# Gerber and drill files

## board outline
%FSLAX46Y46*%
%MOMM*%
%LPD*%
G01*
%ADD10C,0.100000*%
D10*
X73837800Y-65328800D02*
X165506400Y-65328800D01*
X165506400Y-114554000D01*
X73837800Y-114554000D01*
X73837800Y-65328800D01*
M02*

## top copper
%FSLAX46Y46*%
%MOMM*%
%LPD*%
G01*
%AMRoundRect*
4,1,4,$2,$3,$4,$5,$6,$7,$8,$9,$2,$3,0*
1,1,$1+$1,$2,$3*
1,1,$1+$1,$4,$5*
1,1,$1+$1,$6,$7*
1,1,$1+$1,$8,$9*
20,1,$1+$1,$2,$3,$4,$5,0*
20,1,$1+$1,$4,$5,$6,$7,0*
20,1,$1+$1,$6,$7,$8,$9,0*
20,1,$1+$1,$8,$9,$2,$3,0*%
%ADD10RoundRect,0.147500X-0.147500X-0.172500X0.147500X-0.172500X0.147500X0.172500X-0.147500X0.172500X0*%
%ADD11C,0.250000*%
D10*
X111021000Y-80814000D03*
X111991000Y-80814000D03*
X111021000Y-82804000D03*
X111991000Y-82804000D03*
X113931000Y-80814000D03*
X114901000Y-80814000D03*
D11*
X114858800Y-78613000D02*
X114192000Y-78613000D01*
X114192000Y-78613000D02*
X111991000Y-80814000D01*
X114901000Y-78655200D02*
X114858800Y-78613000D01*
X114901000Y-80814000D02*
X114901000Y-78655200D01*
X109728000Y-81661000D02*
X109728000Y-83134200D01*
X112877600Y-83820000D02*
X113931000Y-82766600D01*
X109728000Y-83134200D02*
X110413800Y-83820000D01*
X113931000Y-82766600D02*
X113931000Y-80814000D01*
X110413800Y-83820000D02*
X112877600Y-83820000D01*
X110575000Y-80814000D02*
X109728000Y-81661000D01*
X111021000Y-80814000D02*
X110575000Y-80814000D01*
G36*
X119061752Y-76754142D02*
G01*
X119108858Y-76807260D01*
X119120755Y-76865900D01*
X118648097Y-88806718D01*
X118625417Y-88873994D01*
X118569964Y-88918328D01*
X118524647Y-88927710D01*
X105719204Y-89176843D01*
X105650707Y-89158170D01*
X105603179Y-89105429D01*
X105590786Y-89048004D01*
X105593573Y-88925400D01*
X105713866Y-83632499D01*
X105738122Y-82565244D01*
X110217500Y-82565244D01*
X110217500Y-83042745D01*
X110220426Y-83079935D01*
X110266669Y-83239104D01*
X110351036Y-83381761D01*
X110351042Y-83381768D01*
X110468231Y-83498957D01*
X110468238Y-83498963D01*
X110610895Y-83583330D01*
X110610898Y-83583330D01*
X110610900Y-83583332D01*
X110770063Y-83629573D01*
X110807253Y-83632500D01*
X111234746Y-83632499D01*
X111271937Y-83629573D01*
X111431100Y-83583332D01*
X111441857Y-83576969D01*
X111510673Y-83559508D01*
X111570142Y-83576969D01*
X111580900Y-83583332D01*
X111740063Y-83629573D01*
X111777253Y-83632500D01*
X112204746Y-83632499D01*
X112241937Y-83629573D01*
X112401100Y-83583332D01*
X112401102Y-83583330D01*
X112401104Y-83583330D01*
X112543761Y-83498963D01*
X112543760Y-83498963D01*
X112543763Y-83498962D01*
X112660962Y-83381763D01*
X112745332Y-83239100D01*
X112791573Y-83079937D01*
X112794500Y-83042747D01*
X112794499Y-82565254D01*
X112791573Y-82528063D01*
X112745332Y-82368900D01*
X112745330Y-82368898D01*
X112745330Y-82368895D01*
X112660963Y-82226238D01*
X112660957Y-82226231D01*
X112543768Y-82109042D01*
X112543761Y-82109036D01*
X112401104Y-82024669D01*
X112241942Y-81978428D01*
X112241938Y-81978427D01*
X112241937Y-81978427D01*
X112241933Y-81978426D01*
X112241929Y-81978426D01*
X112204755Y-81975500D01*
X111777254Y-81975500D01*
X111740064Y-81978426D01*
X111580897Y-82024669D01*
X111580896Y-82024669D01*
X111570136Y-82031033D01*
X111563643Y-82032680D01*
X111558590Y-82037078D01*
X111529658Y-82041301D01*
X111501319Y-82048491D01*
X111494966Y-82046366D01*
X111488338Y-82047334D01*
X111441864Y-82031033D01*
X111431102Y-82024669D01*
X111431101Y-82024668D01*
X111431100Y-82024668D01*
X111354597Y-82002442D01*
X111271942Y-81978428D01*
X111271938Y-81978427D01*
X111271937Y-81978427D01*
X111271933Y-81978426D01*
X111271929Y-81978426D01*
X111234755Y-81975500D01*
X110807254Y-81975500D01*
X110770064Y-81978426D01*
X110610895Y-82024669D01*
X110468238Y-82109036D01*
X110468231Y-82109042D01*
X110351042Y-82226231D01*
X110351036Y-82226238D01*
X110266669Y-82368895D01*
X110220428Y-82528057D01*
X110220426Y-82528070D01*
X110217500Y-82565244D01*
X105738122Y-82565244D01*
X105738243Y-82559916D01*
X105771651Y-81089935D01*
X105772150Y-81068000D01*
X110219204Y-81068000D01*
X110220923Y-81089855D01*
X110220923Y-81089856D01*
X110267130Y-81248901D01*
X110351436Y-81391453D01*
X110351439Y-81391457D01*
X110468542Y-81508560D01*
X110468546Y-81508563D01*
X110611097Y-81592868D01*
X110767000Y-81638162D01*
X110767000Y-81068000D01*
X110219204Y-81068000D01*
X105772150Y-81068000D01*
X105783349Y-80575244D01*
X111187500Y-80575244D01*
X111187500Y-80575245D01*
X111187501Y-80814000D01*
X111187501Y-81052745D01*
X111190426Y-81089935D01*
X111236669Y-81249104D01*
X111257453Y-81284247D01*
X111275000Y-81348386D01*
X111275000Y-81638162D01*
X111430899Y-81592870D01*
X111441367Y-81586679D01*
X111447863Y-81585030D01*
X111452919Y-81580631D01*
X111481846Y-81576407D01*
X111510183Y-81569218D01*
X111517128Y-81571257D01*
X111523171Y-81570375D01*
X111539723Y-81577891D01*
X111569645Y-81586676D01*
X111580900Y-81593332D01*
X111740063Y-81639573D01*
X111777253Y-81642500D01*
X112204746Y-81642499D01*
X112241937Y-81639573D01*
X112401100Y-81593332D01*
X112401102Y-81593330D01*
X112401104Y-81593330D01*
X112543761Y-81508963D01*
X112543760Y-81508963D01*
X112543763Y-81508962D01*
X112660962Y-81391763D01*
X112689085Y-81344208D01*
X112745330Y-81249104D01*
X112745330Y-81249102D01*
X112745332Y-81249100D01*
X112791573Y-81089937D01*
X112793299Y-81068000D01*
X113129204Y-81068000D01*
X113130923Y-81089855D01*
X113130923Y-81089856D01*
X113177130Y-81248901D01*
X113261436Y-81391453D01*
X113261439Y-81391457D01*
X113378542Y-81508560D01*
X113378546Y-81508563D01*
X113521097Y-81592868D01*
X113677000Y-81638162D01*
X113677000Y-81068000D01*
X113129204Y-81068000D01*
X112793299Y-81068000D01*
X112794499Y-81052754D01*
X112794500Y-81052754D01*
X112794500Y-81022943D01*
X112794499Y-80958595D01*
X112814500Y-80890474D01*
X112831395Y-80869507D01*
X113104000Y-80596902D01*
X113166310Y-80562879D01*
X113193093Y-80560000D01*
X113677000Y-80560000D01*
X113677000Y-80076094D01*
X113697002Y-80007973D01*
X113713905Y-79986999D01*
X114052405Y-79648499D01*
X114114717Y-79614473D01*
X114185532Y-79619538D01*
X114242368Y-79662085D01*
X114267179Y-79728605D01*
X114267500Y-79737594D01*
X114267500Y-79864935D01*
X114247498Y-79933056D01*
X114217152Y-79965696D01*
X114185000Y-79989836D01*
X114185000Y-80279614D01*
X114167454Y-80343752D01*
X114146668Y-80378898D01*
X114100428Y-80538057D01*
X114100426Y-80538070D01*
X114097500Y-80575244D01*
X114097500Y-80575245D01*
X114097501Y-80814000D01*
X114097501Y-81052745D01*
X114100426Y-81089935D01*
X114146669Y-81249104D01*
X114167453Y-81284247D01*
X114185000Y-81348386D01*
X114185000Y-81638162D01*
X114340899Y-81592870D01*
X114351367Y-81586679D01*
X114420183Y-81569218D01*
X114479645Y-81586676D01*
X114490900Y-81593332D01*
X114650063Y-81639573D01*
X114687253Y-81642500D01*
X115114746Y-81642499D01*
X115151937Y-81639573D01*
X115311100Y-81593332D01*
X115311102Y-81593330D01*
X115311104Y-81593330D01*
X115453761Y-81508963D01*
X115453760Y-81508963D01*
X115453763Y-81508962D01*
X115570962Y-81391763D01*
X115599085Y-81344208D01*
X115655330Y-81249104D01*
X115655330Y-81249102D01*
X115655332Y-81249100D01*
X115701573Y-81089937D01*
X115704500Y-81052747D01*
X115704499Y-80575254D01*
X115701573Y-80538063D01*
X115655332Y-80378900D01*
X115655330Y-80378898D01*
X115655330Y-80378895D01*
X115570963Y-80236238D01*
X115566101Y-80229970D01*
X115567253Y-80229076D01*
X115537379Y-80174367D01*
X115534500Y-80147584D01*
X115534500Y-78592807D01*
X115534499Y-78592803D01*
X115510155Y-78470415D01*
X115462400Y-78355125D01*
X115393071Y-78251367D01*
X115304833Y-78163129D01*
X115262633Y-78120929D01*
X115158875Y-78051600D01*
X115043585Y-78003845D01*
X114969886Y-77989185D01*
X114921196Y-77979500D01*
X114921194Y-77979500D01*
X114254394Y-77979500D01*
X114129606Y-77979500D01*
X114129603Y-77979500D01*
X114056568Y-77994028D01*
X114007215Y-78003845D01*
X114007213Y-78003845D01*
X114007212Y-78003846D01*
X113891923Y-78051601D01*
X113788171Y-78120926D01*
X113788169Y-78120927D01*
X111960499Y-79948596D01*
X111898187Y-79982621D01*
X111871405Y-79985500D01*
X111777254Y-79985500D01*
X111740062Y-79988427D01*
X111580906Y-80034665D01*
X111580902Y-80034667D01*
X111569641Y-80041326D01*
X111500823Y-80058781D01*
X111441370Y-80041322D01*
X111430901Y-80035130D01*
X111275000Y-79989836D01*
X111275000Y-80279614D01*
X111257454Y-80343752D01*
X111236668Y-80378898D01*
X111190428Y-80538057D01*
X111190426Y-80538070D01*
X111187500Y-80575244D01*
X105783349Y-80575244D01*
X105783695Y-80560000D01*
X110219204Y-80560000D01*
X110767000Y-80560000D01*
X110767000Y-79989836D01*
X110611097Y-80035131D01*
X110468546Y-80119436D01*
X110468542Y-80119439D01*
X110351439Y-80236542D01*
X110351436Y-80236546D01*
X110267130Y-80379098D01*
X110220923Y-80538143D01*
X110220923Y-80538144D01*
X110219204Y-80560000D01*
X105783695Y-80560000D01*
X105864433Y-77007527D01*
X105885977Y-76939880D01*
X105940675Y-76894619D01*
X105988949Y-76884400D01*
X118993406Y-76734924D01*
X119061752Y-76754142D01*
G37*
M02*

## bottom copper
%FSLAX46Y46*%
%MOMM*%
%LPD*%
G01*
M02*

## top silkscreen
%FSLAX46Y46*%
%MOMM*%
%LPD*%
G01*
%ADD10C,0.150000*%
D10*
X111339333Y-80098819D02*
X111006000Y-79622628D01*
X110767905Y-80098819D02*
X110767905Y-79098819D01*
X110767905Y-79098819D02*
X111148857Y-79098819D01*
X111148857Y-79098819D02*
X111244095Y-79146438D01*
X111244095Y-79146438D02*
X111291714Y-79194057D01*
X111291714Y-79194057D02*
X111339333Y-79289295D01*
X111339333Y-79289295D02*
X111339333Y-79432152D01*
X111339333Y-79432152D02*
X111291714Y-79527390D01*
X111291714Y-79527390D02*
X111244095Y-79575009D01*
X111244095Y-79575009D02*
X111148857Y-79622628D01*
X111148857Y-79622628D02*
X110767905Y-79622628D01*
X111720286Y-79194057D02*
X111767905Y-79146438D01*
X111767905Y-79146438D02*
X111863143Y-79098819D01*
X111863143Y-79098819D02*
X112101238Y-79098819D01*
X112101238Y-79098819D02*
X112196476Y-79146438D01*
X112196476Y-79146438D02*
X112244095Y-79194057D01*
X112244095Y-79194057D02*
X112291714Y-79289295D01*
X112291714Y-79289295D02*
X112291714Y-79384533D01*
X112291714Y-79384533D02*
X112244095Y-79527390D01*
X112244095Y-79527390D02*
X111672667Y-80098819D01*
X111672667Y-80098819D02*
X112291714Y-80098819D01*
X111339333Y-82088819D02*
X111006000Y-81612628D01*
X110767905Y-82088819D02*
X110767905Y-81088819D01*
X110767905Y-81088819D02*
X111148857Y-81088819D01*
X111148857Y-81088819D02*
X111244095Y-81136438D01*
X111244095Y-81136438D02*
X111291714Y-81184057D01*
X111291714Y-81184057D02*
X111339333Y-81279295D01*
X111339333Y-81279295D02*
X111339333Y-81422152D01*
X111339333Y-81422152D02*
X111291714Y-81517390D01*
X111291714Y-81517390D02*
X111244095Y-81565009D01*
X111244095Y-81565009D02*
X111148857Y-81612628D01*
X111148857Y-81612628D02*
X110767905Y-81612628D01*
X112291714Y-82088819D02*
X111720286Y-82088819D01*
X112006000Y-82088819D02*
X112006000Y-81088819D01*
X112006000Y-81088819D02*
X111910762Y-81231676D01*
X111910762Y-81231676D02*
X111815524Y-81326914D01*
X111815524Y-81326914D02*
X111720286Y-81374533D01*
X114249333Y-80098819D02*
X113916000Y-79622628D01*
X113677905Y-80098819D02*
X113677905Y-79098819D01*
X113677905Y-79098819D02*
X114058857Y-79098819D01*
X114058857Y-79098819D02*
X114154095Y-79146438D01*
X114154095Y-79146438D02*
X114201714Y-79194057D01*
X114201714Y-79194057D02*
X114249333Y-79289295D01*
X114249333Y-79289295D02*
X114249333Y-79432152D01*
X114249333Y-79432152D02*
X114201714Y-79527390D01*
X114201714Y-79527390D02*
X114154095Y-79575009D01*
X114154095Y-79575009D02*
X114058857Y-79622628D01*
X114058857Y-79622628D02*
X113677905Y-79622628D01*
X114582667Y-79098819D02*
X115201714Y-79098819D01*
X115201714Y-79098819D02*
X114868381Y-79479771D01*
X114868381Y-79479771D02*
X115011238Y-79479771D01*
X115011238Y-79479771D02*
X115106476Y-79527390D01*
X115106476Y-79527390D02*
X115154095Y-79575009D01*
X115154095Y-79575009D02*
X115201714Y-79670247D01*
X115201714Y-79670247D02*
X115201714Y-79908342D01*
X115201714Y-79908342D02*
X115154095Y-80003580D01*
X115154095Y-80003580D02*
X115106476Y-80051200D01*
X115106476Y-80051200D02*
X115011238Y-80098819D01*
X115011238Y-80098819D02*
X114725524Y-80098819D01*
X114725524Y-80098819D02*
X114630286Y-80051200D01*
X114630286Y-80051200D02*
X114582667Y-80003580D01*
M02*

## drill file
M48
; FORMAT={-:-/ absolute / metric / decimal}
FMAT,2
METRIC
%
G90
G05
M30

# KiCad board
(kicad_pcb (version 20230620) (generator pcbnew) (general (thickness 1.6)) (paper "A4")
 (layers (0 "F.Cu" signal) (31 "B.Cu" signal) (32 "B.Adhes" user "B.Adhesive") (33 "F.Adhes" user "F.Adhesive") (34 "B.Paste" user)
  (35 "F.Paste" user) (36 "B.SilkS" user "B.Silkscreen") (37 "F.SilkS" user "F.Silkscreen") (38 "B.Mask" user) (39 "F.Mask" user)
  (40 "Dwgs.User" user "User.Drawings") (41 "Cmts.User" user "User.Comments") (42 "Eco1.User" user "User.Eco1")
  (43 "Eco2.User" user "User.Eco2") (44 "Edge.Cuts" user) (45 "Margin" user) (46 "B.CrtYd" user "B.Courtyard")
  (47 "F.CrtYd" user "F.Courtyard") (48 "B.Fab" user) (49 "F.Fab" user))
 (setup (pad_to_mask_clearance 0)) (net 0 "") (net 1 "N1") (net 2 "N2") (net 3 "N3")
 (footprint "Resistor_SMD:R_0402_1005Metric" (layer "F.Cu") (at 111.506 80.814)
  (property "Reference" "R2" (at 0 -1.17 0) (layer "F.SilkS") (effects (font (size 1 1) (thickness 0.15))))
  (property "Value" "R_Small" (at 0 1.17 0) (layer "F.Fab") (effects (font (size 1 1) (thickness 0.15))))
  (pad "1" smd roundrect (at -0.485 0) (size 0.59 0.64) (layers "F.Cu" "F.Paste" "F.Mask") (roundrect_rratio 0.25) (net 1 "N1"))
  (pad "2" smd roundrect (at 0.485 0) (size 0.59 0.64) (layers "F.Cu" "F.Paste" "F.Mask") (roundrect_rratio 0.25) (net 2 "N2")))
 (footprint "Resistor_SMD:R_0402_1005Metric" (layer "F.Cu") (at 111.506 82.804)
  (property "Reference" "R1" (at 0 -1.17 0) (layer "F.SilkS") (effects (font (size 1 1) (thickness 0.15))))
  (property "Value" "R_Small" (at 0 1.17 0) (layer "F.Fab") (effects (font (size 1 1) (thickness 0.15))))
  (pad "1" smd roundrect (at -0.485 0) (size 0.59 0.64) (layers "F.Cu" "F.Paste" "F.Mask") (roundrect_rratio 0.25) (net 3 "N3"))
  (pad "2" smd roundrect (at 0.485 0) (size 0.59 0.64) (layers "F.Cu" "F.Paste" "F.Mask") (roundrect_rratio 0.25) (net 2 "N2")))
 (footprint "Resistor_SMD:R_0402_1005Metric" (layer "F.Cu") (at 114.416 80.814)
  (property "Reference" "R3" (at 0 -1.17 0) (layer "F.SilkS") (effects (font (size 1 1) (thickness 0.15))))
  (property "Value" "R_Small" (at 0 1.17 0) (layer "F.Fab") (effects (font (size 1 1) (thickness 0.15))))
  (pad "1" smd roundrect (at -0.485 0) (size 0.59 0.64) (layers "F.Cu" "F.Paste" "F.Mask") (roundrect_rratio 0.25) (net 1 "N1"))
  (pad "2" smd roundrect (at 0.485 0) (size 0.59 0.64) (layers "F.Cu" "F.Paste" "F.Mask") (roundrect_rratio 0.25) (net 2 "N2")))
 (gr_rect (start 73.8378 65.3288) (end 165.5064 114.554) (stroke (width 0.1) (type solid)) (fill none) (layer "Edge.Cuts"))
 (segment (start 114.8588 78.613) (end 114.192 78.613) (width 0.25) (layer "F.Cu") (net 2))
 (segment (start 114.192 78.613) (end 111.991 80.814) (width 0.25) (layer "F.Cu") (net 2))
 (segment (start 114.901 78.6552) (end 114.8588 78.613) (width 0.25) (layer "F.Cu") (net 2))
 (segment (start 114.901 80.814) (end 114.901 78.6552) (width 0.25) (layer "F.Cu") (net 2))
 (segment (start 109.728 81.661) (end 109.728 83.1342) (width 0.25) (layer "F.Cu") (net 1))
 (segment (start 112.8776 83.82) (end 113.931 82.7666) (width 0.25) (layer "F.Cu") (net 1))
 (segment (start 109.728 83.1342) (end 110.4138 83.82) (width 0.25) (layer "F.Cu") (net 1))
 (segment (start 113.931 82.7666) (end 113.931 80.814) (width 0.25) (layer "F.Cu") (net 1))
 (segment (start 110.4138 83.82) (end 112.8776 83.82) (width 0.25) (layer "F.Cu") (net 1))
 (segment (start 110.575 80.814) (end 109.728 81.661) (width 0.25) (layer "F.Cu") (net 1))
 (segment (start 111.021 80.814) (end 110.575 80.814) (width 0.25) (layer "F.Cu") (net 1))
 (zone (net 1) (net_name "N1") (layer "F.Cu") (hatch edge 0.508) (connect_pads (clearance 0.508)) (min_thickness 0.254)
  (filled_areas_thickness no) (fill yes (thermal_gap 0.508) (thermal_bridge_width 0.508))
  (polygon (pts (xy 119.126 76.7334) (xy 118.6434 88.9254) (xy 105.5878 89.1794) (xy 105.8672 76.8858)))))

